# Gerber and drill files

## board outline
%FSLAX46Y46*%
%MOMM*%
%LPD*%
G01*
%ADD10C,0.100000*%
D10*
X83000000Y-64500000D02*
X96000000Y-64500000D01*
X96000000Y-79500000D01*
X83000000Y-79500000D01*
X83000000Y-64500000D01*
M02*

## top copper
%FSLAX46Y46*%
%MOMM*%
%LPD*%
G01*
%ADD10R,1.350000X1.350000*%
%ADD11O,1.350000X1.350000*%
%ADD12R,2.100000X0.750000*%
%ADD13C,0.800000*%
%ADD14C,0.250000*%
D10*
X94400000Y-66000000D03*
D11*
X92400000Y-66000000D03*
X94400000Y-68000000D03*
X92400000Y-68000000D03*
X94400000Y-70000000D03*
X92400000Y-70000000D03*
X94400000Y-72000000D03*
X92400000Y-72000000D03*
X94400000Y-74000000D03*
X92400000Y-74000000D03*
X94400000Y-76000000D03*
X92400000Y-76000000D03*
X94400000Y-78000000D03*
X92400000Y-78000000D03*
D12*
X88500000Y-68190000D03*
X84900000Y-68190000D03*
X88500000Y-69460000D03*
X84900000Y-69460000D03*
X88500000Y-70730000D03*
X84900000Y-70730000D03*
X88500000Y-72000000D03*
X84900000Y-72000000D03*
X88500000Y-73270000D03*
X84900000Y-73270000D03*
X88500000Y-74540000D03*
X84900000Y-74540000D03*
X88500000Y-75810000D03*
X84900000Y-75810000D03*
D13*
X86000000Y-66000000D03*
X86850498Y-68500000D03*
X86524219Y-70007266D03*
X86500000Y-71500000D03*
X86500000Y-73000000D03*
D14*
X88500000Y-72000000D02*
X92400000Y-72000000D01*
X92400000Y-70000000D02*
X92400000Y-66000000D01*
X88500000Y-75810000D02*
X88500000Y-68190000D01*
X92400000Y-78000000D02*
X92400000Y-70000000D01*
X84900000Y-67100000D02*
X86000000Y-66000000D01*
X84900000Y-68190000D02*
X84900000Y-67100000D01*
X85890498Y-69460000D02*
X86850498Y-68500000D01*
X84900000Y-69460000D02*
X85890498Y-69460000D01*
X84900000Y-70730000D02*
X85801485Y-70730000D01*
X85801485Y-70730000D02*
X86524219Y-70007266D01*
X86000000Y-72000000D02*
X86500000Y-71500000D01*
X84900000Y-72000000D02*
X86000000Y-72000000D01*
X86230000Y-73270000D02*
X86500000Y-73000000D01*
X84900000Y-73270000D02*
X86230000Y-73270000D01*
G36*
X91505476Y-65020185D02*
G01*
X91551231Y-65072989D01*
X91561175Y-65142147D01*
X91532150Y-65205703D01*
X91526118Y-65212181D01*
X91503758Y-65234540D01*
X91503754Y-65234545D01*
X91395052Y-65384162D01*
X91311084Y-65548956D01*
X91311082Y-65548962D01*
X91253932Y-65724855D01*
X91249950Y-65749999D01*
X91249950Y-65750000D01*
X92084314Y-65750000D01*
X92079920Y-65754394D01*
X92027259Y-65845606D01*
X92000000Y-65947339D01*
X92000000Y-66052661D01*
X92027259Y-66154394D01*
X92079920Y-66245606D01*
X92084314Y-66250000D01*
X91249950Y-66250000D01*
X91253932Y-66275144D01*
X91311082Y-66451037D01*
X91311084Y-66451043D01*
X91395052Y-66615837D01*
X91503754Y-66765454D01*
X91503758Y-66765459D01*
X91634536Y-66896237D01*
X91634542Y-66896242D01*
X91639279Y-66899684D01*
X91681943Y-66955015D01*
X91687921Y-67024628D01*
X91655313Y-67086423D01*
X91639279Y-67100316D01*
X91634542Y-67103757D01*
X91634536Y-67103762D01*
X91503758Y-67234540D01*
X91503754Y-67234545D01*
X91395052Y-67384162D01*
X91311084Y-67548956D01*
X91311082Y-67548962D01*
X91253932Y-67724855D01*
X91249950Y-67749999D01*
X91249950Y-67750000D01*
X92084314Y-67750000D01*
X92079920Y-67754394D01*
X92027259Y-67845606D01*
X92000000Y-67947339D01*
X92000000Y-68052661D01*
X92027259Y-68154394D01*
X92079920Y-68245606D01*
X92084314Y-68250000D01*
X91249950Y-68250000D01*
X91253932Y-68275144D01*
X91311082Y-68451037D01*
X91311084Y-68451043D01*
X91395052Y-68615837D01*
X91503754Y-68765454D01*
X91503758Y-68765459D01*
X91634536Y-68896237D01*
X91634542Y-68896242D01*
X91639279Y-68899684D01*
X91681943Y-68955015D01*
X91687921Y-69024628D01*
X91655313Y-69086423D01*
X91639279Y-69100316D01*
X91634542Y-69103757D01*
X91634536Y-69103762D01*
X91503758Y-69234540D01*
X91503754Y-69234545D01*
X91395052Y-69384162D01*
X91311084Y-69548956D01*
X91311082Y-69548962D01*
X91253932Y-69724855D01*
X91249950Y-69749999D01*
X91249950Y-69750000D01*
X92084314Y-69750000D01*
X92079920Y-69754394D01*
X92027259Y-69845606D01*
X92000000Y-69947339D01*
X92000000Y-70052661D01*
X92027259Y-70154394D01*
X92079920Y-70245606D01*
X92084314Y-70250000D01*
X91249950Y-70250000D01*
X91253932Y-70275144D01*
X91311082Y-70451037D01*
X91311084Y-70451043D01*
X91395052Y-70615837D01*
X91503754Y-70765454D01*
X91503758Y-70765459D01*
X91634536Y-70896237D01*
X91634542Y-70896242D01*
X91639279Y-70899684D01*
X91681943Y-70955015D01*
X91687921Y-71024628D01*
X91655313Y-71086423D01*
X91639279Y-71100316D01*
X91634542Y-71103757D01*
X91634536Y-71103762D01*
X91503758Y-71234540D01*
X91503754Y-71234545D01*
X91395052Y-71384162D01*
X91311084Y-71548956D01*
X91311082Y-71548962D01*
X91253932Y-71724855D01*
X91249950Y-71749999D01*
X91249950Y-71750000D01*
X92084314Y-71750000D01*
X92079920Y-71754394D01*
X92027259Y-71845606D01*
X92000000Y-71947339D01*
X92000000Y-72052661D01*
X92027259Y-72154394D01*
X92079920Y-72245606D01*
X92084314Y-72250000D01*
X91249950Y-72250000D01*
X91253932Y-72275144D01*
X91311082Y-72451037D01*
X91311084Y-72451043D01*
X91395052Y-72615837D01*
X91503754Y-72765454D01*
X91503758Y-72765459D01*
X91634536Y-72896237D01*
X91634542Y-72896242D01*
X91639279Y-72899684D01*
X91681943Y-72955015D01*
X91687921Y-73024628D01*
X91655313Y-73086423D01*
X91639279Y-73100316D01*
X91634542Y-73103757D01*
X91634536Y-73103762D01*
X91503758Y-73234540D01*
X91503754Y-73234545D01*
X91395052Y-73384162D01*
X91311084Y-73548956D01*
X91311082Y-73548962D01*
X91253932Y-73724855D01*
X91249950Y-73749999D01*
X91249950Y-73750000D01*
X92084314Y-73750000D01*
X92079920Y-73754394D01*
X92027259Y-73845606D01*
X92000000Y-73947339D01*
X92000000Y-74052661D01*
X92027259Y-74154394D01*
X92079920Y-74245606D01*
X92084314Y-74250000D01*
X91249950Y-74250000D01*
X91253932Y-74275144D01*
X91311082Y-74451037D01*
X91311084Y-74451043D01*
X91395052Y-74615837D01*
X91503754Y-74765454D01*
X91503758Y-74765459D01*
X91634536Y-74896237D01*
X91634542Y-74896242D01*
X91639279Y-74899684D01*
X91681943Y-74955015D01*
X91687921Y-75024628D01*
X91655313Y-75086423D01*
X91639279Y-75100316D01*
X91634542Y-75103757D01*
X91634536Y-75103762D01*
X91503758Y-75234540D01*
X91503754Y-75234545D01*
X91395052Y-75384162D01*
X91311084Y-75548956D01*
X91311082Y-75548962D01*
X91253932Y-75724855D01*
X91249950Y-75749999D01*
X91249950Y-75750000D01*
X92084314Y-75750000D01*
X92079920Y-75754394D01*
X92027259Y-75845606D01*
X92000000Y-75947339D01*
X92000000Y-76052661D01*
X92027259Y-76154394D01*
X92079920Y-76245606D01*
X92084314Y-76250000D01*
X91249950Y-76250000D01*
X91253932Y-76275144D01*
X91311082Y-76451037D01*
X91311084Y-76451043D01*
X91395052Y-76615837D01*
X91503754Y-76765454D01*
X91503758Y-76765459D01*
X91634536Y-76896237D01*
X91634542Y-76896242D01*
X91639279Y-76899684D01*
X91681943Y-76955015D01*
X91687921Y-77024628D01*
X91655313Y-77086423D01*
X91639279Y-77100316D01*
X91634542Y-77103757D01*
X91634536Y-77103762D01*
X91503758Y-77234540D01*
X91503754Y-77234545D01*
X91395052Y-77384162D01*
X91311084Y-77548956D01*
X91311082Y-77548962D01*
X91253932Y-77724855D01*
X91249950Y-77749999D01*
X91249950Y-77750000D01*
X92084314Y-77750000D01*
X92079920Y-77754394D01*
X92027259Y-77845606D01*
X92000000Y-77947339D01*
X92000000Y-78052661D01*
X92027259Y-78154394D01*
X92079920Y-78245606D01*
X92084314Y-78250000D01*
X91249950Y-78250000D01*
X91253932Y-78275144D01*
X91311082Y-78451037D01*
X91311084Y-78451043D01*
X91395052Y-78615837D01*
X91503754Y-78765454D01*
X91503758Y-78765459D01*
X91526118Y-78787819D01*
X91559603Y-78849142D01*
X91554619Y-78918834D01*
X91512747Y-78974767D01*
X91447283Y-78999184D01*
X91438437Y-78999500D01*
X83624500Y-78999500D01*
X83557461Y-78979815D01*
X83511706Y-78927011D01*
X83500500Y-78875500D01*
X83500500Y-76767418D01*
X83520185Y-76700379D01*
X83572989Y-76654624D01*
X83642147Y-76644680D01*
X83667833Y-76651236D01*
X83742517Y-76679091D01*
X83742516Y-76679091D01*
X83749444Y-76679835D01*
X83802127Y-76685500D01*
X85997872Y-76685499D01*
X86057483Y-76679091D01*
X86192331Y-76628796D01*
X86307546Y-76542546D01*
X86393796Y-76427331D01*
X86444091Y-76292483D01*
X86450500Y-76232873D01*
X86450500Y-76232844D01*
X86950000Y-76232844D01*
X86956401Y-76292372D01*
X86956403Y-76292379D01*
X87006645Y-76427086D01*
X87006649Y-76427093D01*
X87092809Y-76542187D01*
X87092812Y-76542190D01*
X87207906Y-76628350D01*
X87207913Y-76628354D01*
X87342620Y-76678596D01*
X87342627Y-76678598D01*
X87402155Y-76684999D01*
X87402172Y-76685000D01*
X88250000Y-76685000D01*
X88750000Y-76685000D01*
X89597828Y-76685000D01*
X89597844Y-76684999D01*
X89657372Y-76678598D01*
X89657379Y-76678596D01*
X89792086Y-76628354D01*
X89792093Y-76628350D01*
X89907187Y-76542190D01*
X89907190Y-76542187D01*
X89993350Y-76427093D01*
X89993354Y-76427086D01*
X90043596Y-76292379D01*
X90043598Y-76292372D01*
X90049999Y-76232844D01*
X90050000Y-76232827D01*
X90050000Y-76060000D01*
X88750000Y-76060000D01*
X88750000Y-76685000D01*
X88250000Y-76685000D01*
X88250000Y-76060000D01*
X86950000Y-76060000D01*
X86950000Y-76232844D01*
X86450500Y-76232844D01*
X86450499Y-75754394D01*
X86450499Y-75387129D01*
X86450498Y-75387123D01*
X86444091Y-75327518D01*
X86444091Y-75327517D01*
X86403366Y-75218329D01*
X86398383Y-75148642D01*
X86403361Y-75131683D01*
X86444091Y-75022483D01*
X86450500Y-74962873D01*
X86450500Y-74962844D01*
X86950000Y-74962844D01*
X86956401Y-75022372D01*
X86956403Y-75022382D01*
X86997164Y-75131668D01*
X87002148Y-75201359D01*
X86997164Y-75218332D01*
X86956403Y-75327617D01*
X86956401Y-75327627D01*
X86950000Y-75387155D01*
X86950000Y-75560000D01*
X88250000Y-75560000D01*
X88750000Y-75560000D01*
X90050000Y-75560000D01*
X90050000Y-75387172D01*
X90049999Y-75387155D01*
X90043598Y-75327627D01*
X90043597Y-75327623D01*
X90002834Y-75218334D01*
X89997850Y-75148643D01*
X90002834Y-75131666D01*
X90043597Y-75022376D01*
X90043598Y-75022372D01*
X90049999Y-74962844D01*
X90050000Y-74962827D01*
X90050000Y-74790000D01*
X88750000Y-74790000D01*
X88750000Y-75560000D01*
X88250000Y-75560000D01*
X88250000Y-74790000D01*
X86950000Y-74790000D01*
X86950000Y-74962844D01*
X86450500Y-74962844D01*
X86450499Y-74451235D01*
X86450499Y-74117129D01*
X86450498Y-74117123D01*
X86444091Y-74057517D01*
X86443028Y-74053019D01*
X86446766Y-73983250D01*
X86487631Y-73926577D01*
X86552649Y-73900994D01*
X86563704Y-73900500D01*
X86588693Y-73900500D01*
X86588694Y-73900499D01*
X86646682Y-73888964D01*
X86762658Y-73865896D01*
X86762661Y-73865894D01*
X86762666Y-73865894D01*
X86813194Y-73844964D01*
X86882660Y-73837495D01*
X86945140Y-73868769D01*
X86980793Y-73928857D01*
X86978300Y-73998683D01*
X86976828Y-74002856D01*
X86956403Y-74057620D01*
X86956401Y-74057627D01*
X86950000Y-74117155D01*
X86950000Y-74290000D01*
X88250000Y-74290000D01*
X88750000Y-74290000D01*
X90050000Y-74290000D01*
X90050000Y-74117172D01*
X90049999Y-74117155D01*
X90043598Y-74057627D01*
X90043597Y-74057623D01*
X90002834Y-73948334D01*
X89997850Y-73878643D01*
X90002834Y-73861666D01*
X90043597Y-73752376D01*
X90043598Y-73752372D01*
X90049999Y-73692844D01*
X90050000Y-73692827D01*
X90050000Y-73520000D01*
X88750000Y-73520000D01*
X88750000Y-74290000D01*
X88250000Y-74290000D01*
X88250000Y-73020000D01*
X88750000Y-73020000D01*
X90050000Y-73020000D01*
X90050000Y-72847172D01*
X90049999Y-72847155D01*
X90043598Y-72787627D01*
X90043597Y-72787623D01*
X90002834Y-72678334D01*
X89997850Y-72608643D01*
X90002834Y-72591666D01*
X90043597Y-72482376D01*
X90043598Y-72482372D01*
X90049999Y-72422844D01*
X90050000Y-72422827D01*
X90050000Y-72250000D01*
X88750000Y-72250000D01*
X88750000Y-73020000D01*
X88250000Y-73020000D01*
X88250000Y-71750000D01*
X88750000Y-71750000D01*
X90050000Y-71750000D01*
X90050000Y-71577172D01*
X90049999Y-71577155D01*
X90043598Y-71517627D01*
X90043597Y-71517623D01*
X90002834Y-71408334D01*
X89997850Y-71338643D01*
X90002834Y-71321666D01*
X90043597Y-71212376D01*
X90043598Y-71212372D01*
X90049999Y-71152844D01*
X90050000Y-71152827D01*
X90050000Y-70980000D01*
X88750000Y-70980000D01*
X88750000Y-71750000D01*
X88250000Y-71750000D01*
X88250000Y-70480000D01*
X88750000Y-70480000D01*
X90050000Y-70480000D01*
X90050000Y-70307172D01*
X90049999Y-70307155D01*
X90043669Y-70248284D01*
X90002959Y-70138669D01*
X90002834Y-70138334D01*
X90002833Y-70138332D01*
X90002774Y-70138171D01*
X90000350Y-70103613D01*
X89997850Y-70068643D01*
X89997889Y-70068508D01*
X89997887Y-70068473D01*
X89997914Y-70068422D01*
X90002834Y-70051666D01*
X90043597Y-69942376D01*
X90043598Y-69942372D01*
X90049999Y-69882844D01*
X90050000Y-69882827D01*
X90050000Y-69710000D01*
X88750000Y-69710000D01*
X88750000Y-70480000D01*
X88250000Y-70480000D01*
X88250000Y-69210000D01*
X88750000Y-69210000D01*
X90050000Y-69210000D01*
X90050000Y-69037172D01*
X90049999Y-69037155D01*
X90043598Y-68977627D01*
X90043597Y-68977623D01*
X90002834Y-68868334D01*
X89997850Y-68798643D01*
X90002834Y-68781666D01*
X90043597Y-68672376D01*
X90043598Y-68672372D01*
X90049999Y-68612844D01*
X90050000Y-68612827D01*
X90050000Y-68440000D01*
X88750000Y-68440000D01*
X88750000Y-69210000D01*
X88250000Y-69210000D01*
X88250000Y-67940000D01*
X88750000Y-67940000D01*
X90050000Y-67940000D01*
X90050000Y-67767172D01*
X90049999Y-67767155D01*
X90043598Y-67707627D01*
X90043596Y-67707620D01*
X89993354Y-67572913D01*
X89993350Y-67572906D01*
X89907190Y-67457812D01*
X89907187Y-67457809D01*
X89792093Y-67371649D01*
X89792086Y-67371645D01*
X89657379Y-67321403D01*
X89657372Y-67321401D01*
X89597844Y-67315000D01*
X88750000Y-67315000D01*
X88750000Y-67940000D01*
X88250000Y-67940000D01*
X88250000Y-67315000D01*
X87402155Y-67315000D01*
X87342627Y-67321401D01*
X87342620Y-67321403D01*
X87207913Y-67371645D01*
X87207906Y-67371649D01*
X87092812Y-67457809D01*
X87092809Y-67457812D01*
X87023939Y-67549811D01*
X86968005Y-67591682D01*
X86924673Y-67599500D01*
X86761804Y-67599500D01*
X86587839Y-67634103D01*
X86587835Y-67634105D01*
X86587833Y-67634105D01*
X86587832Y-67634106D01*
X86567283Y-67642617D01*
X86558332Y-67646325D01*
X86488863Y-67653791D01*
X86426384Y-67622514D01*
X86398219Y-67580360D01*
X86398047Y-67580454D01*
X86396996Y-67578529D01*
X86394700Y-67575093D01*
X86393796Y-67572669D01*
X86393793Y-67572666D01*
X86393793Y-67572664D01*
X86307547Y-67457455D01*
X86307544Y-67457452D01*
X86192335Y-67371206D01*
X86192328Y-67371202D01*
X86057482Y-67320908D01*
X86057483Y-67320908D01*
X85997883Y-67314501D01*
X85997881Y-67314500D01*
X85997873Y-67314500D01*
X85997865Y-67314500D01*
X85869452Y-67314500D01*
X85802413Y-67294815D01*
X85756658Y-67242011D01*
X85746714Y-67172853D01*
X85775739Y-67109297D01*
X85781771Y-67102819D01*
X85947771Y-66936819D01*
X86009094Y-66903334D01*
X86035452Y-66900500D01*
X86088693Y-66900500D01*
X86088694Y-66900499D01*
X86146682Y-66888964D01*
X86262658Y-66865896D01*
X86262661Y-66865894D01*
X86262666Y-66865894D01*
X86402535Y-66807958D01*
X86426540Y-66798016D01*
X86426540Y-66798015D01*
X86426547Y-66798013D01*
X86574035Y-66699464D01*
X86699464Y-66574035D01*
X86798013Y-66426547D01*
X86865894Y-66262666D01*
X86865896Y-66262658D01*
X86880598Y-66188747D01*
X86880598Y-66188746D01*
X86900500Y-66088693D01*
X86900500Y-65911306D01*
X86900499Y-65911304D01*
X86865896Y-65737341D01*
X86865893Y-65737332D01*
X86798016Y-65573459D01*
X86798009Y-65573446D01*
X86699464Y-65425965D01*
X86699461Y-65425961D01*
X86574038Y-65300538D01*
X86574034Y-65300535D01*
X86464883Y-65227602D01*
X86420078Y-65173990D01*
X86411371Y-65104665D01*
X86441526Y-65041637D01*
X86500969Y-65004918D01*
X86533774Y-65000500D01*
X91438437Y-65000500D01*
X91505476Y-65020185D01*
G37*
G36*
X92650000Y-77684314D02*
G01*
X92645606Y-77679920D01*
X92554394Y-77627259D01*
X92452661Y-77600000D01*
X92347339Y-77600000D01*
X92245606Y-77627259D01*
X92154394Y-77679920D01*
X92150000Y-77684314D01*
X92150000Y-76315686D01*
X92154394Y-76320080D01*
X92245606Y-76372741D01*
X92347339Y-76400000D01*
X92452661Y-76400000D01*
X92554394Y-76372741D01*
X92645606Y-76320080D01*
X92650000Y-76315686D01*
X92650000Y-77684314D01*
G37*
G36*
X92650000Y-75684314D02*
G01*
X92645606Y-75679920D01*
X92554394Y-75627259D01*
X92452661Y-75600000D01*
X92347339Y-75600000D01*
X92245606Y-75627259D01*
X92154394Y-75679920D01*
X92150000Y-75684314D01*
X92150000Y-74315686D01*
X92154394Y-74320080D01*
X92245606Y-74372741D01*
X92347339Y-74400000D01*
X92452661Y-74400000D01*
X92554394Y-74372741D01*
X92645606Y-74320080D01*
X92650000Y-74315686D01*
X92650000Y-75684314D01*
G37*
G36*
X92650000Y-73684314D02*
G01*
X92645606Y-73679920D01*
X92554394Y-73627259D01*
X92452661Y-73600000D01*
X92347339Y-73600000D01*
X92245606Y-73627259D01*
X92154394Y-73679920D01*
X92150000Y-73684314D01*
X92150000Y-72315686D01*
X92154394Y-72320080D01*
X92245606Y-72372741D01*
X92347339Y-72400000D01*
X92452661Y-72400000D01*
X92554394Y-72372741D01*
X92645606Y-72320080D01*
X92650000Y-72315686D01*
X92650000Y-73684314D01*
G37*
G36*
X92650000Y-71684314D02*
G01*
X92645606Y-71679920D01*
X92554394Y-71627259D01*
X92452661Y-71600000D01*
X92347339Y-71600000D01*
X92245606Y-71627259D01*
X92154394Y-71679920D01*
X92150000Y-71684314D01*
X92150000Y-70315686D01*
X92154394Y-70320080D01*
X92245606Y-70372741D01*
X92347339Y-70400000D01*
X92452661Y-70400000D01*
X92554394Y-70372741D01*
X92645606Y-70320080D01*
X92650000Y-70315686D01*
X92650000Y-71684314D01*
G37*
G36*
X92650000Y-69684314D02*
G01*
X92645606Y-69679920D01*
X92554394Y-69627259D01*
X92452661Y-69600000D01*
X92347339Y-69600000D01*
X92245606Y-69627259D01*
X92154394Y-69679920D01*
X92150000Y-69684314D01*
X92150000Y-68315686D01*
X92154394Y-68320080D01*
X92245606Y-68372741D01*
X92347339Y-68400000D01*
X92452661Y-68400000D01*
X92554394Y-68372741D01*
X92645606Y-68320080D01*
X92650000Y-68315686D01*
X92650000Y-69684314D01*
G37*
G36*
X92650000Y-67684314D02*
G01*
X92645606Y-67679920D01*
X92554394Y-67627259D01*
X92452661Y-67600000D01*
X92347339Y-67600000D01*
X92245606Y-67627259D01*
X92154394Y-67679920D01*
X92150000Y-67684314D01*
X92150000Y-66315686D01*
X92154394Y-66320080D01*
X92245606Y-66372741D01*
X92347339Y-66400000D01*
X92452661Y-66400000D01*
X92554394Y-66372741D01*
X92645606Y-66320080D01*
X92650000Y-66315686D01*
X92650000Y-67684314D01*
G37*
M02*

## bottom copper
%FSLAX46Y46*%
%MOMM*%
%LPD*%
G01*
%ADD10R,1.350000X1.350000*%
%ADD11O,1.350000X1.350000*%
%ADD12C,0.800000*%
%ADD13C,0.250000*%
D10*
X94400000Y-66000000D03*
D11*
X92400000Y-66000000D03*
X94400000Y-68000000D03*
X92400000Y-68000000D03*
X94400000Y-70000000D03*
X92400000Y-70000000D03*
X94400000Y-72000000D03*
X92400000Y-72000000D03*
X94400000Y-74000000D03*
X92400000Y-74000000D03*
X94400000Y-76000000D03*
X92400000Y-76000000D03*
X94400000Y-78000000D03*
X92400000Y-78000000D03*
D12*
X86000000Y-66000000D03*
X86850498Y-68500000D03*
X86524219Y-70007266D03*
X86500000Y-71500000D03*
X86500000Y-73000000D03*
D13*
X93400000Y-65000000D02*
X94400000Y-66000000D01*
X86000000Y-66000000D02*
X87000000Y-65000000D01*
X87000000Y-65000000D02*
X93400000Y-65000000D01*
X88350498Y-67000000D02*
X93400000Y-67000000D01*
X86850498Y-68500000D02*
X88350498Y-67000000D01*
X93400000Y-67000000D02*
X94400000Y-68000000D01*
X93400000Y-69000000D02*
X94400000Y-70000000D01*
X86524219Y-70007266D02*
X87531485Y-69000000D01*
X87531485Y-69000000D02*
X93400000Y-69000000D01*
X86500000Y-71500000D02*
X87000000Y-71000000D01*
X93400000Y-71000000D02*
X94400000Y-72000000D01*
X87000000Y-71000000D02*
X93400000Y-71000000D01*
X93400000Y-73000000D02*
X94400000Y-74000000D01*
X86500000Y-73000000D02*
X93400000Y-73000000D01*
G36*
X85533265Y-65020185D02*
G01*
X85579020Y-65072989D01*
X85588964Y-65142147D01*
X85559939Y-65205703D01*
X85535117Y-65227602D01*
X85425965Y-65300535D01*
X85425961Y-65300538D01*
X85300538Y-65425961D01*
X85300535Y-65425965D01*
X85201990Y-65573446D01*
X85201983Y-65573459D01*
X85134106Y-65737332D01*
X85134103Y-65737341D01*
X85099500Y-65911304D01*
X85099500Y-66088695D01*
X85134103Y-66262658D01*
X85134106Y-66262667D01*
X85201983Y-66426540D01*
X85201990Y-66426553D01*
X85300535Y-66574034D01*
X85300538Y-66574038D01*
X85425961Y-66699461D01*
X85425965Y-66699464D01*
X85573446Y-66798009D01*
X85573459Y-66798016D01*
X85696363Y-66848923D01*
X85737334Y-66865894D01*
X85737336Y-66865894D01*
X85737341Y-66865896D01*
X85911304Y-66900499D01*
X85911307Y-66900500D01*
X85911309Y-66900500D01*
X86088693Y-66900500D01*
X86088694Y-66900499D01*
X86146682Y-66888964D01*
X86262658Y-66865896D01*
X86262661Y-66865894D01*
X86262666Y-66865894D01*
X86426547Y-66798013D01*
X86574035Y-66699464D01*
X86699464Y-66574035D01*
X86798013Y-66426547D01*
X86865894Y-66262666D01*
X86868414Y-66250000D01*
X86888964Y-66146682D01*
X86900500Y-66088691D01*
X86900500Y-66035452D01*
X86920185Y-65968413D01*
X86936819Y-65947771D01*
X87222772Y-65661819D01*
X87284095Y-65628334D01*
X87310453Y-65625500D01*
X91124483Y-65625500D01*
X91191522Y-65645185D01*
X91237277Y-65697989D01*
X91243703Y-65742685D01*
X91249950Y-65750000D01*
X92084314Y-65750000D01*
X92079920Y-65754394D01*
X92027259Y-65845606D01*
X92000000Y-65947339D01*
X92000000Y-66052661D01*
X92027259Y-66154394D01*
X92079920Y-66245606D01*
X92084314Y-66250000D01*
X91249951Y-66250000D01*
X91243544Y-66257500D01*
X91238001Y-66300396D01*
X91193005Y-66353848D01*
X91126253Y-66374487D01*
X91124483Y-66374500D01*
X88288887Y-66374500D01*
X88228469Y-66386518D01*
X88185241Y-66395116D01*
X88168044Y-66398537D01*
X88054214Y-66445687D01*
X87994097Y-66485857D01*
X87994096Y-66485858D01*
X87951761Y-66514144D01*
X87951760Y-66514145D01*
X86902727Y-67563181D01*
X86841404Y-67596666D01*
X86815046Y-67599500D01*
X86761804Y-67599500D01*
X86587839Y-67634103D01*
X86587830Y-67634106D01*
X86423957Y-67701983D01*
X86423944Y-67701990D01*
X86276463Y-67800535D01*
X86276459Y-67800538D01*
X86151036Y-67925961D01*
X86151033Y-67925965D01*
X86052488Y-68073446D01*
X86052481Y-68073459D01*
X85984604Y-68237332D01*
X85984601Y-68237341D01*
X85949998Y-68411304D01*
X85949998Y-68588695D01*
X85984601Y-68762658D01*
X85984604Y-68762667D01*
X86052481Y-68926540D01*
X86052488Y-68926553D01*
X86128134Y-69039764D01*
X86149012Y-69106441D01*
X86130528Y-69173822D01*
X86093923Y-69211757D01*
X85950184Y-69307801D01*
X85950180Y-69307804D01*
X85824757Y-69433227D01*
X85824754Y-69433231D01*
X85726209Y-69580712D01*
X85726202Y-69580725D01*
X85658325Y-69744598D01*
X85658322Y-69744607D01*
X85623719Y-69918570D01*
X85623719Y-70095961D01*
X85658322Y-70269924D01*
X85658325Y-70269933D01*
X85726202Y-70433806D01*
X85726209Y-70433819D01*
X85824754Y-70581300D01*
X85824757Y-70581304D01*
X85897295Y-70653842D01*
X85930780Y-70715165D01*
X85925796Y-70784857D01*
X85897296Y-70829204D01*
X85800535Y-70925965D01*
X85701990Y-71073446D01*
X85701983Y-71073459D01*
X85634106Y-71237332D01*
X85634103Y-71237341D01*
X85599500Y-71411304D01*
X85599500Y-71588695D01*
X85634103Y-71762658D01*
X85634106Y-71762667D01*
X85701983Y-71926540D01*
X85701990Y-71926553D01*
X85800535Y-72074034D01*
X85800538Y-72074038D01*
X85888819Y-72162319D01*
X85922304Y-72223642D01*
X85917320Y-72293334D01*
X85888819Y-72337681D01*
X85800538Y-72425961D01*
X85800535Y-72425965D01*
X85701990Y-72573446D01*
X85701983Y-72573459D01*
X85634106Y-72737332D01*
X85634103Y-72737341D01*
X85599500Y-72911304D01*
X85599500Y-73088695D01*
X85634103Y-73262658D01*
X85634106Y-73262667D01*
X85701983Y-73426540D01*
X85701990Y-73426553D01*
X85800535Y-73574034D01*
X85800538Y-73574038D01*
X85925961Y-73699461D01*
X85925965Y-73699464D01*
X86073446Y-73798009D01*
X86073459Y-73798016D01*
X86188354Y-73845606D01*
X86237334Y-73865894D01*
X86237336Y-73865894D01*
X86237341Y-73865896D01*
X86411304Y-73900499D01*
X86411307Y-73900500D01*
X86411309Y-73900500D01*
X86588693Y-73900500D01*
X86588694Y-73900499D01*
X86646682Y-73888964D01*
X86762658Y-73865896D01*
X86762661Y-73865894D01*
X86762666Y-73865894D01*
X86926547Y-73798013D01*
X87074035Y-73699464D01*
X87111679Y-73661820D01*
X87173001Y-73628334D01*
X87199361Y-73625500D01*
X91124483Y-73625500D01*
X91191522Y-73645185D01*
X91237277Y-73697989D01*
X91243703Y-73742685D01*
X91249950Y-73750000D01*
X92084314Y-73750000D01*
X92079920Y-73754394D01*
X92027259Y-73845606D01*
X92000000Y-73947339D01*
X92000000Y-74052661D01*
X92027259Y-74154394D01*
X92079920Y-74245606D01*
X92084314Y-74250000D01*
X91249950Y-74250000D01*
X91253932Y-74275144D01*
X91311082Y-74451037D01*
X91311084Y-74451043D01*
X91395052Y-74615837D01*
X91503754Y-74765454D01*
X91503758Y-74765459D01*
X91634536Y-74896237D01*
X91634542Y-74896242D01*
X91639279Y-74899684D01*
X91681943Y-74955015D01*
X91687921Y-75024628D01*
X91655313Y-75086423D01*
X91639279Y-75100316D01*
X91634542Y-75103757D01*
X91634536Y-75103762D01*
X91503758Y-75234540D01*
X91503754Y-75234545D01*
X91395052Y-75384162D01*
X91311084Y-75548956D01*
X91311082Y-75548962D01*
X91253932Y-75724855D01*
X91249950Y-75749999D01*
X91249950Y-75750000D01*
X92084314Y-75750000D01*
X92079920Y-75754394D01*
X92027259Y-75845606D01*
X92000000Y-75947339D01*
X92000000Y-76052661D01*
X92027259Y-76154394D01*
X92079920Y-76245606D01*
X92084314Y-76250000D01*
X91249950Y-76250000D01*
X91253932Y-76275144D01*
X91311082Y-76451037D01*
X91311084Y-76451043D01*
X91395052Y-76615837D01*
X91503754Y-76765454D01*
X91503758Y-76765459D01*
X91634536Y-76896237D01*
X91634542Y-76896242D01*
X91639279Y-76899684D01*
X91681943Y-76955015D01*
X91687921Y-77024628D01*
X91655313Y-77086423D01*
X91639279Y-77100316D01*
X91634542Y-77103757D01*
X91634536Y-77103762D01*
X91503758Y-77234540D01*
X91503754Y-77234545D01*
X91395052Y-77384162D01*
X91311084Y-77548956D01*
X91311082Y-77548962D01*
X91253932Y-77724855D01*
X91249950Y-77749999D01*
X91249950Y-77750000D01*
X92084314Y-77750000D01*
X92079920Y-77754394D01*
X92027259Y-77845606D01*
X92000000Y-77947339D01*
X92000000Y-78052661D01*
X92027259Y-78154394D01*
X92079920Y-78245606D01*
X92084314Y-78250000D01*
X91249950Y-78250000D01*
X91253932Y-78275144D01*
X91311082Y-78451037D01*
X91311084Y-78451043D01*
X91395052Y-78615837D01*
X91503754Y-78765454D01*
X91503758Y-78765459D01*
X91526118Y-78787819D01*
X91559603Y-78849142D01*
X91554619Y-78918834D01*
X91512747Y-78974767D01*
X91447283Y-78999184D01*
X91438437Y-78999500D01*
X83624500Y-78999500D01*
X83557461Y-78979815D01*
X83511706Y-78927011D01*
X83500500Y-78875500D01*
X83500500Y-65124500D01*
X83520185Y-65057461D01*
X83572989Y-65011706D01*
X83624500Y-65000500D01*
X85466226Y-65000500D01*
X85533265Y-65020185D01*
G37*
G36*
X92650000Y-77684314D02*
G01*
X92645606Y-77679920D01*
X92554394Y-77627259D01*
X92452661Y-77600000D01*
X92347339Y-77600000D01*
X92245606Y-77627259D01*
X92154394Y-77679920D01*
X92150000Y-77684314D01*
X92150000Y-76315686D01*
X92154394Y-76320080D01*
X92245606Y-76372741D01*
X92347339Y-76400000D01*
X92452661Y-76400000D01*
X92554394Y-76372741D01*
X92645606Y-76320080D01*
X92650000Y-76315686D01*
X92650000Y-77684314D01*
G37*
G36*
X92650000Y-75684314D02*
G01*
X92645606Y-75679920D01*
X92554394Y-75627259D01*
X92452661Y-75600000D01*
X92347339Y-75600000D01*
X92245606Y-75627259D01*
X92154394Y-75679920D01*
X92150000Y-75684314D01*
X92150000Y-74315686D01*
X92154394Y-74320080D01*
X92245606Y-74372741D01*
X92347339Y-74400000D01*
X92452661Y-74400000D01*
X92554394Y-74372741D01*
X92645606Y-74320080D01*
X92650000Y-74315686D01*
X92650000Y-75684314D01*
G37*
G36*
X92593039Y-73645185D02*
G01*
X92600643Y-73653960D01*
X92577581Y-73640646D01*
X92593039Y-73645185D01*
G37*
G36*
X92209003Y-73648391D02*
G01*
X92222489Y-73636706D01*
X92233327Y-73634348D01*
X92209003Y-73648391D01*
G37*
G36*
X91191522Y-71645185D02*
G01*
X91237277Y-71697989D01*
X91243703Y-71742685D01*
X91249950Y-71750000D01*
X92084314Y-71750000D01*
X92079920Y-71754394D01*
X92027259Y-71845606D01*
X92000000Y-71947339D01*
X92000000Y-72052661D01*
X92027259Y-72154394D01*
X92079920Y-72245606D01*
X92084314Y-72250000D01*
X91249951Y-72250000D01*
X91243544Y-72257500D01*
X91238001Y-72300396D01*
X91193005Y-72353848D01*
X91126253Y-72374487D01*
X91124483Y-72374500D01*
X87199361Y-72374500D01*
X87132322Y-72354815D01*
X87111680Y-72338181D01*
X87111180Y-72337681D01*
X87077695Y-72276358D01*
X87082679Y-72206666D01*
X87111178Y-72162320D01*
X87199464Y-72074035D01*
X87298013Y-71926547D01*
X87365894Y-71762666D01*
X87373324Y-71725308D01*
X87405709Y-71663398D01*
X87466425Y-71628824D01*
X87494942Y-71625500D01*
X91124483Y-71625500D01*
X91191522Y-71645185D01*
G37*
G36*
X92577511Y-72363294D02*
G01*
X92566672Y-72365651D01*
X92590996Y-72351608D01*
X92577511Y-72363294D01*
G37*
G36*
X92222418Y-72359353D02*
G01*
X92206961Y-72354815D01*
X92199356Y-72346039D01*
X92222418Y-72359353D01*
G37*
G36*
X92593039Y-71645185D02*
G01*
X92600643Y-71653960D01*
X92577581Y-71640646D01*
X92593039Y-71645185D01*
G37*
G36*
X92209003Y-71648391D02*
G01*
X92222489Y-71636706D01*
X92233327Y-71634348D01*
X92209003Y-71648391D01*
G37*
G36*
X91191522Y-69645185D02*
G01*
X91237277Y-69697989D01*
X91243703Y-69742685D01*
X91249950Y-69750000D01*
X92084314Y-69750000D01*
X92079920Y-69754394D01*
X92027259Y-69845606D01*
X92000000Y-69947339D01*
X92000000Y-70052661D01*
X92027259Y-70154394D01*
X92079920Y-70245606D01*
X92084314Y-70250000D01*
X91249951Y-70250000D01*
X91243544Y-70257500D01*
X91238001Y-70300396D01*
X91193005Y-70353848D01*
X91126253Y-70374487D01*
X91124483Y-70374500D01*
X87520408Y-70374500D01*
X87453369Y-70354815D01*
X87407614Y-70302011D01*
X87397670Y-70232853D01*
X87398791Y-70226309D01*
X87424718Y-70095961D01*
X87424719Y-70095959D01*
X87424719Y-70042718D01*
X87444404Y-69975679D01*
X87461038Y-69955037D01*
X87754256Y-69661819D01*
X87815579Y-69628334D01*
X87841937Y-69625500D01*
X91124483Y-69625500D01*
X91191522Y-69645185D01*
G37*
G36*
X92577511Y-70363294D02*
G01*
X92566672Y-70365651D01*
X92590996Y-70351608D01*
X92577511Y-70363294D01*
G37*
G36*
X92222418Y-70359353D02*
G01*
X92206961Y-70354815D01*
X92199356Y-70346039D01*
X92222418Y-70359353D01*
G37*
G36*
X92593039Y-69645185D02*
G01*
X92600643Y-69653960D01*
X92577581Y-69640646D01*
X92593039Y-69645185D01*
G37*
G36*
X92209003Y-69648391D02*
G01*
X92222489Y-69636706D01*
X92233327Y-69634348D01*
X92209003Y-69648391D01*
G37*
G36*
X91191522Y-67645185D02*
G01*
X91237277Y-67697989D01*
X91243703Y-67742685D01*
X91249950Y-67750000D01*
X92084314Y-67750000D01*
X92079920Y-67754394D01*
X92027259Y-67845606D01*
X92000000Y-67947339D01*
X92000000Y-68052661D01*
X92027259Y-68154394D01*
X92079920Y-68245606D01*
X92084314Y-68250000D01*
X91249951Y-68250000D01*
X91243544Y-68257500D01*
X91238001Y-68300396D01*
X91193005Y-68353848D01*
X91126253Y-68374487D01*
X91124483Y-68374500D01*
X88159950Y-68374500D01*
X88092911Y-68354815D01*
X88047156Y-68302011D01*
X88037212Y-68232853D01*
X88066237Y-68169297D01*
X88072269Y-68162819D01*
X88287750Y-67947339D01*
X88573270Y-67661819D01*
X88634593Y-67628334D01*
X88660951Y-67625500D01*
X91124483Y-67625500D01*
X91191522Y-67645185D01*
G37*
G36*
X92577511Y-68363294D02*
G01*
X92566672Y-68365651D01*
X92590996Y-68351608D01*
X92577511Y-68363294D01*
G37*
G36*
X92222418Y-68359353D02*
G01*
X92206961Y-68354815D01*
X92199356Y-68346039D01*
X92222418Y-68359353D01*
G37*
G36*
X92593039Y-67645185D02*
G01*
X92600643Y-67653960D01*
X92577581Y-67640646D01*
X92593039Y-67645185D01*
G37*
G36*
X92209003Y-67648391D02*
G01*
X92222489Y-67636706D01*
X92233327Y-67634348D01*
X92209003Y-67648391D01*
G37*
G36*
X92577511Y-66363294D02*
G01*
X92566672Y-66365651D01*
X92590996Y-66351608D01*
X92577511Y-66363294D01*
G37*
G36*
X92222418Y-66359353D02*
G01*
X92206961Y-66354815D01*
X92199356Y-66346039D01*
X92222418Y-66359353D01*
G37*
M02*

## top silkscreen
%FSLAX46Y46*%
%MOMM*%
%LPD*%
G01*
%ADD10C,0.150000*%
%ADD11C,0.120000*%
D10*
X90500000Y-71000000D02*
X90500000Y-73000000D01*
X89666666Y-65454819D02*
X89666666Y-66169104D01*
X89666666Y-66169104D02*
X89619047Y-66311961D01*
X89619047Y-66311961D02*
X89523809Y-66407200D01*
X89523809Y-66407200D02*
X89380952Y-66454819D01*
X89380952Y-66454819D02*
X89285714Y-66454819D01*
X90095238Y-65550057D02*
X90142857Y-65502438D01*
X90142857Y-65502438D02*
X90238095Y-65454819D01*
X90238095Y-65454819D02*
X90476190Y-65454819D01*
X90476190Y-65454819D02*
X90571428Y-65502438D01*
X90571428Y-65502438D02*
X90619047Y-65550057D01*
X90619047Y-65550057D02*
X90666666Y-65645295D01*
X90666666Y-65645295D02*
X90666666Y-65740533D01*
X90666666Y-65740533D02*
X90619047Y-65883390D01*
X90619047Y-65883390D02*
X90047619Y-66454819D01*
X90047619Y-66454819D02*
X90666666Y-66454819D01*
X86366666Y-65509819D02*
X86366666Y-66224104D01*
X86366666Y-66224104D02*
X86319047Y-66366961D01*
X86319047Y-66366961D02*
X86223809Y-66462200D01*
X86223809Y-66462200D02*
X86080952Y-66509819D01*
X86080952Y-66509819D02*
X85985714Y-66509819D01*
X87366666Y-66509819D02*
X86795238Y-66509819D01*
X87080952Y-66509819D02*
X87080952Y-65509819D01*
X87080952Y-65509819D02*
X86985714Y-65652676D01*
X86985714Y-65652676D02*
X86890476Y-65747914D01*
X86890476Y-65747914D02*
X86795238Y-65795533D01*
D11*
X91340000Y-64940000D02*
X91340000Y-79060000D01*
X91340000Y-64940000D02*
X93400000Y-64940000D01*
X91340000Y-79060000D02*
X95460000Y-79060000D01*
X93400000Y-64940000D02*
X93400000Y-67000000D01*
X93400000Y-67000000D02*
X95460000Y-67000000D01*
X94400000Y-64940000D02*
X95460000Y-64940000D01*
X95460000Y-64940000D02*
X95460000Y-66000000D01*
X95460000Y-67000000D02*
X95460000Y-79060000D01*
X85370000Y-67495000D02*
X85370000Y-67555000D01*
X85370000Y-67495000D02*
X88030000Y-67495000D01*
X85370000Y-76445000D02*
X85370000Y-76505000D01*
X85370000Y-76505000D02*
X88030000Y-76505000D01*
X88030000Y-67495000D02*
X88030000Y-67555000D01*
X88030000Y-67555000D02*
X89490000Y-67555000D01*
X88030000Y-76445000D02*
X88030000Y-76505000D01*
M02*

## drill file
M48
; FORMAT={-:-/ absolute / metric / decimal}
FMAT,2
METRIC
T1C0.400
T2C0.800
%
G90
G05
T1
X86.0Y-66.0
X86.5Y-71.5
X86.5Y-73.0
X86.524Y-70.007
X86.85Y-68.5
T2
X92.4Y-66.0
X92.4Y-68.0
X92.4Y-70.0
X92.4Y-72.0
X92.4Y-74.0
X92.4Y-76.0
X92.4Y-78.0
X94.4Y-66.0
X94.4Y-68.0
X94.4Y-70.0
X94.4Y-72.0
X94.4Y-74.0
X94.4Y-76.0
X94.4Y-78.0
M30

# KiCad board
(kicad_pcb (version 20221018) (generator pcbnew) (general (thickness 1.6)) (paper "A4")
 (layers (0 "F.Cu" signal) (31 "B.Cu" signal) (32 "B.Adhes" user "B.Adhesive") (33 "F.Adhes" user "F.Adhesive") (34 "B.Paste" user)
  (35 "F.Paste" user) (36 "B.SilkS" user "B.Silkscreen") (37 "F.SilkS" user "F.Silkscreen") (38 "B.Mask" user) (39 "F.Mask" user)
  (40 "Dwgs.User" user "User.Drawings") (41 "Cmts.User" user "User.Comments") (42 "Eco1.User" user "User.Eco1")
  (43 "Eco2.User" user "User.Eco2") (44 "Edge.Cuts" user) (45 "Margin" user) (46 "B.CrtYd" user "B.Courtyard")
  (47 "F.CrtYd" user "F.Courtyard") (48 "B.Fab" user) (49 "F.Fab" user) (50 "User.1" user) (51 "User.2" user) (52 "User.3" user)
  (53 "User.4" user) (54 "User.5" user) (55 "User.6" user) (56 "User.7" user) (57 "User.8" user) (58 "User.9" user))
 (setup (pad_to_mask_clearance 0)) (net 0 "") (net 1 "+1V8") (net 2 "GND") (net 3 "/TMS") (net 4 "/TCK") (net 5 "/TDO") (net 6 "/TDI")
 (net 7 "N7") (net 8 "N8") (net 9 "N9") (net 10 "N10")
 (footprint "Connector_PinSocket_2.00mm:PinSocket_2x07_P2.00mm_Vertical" (layer "F.Cu") (at 94.4 66)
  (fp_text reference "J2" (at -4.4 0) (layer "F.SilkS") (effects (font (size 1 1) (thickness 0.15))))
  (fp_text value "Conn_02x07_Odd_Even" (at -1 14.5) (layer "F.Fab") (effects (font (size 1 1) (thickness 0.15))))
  (fp_line (start -3.06 -1.06) (end -3.06 13.06) (stroke (width 0.12) (type solid)) (layer "F.SilkS"))
  (fp_line (start -3.06 -1.06) (end -1 -1.06) (stroke (width 0.12) (type solid)) (layer "F.SilkS"))
  (fp_line (start -3.06 13.06) (end 1.06 13.06) (stroke (width 0.12) (type solid)) (layer "F.SilkS"))
  (fp_line (start -1 -1.06) (end -1 1) (stroke (width 0.12) (type solid)) (layer "F.SilkS"))
  (fp_line (start -1 1) (end 1.06 1) (stroke (width 0.12) (type solid)) (layer "F.SilkS"))
  (fp_line (start 0 -1.06) (end 1.06 -1.06) (stroke (width 0.12) (type solid)) (layer "F.SilkS"))
  (fp_line (start 1.06 -1.06) (end 1.06 0) (stroke (width 0.12) (type solid)) (layer "F.SilkS"))
  (fp_line (start 1.06 1) (end 1.06 13.06) (stroke (width 0.12) (type solid)) (layer "F.SilkS"))
  (pad "1" thru_hole rect (at 0 0) (size 1.35 1.35) (drill 0.8) (layers "*.Cu" "*.Mask") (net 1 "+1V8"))
  (pad "2" thru_hole oval (at -2 0) (size 1.35 1.35) (drill 0.8) (layers "*.Cu" "*.Mask") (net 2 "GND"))
  (pad "3" thru_hole oval (at 0 2) (size 1.35 1.35) (drill 0.8) (layers "*.Cu" "*.Mask") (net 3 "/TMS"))
  (pad "4" thru_hole oval (at -2 2) (size 1.35 1.35) (drill 0.8) (layers "*.Cu" "*.Mask") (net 2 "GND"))
  (pad "5" thru_hole oval (at 0 4) (size 1.35 1.35) (drill 0.8) (layers "*.Cu" "*.Mask") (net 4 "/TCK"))
  (pad "6" thru_hole oval (at -2 4) (size 1.35 1.35) (drill 0.8) (layers "*.Cu" "*.Mask") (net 2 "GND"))
  (pad "7" thru_hole oval (at 0 6) (size 1.35 1.35) (drill 0.8) (layers "*.Cu" "*.Mask") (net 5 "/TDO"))
  (pad "8" thru_hole oval (at -2 6) (size 1.35 1.35) (drill 0.8) (layers "*.Cu" "*.Mask") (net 2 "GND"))
  (pad "9" thru_hole oval (at 0 8) (size 1.35 1.35) (drill 0.8) (layers "*.Cu" "*.Mask") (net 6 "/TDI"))
  (pad "10" thru_hole oval (at -2 8) (size 1.35 1.35) (drill 0.8) (layers "*.Cu" "*.Mask") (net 2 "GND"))
  (pad "11" thru_hole oval (at 0 10) (size 1.35 1.35) (drill 0.8) (layers "*.Cu" "*.Mask") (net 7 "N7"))
  (pad "12" thru_hole oval (at -2 10) (size 1.35 1.35) (drill 0.8) (layers "*.Cu" "*.Mask") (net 2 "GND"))
  (pad "13" thru_hole oval (at 0 12) (size 1.35 1.35) (drill 0.8) (layers "*.Cu" "*.Mask") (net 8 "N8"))
  (pad "14" thru_hole oval (at -2 12) (size 1.35 1.35) (drill 0.8) (layers "*.Cu" "*.Mask") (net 2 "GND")))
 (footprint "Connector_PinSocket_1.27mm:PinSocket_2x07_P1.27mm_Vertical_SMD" (layer "F.Cu") (at 86.7 72)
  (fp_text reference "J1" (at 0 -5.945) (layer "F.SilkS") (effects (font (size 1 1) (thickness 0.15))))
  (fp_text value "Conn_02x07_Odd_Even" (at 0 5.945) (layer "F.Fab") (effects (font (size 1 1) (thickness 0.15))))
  (fp_line (start -1.33 -4.505) (end -1.33 -4.445) (stroke (width 0.12) (type solid)) (layer "F.SilkS"))
  (fp_line (start -1.33 -4.505) (end 1.33 -4.505) (stroke (width 0.12) (type solid)) (layer "F.SilkS"))
  (fp_line (start -1.33 4.445) (end -1.33 4.505) (stroke (width 0.12) (type solid)) (layer "F.SilkS"))
  (fp_line (start -1.33 4.505) (end 1.33 4.505) (stroke (width 0.12) (type solid)) (layer "F.SilkS"))
  (fp_line (start 1.33 -4.505) (end 1.33 -4.445) (stroke (width 0.12) (type solid)) (layer "F.SilkS"))
  (fp_line (start 1.33 -4.445) (end 2.79 -4.445) (stroke (width 0.12) (type solid)) (layer "F.SilkS"))
  (fp_line (start 1.33 4.445) (end 1.33 4.505) (stroke (width 0.12) (type solid)) (layer "F.SilkS"))
  (pad "1" smd rect (at 1.8 -3.81) (size 2.1 0.75) (layers "F.Cu" "F.Paste" "F.Mask") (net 2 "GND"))
  (pad "2" smd rect (at -1.8 -3.81) (size 2.1 0.75) (layers "F.Cu" "F.Paste" "F.Mask") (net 1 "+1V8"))
  (pad "3" smd rect (at 1.8 -2.54) (size 2.1 0.75) (layers "F.Cu" "F.Paste" "F.Mask") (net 2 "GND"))
  (pad "4" smd rect (at -1.8 -2.54) (size 2.1 0.75) (layers "F.Cu" "F.Paste" "F.Mask") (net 3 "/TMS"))
  (pad "5" smd rect (at 1.8 -1.27) (size 2.1 0.75) (layers "F.Cu" "F.Paste" "F.Mask") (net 2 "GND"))
  (pad "6" smd rect (at -1.8 -1.27) (size 2.1 0.75) (layers "F.Cu" "F.Paste" "F.Mask") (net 4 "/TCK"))
  (pad "7" smd rect (at 1.8 0) (size 2.1 0.75) (layers "F.Cu" "F.Paste" "F.Mask") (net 2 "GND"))
  (pad "8" smd rect (at -1.8 0) (size 2.1 0.75) (layers "F.Cu" "F.Paste" "F.Mask") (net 5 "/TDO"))
  (pad "9" smd rect (at 1.8 1.27) (size 2.1 0.75) (layers "F.Cu" "F.Paste" "F.Mask") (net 2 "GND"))
  (pad "10" smd rect (at -1.8 1.27) (size 2.1 0.75) (layers "F.Cu" "F.Paste" "F.Mask") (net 6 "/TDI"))
  (pad "11" smd rect (at 1.8 2.54) (size 2.1 0.75) (layers "F.Cu" "F.Paste" "F.Mask") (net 2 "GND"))
  (pad "12" smd rect (at -1.8 2.54) (size 2.1 0.75) (layers "F.Cu" "F.Paste" "F.Mask") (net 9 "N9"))
  (pad "13" smd rect (at 1.8 3.81) (size 2.1 0.75) (layers "F.Cu" "F.Paste" "F.Mask") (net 2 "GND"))
  (pad "14" smd rect (at -1.8 3.81) (size 2.1 0.75) (layers "F.Cu" "F.Paste" "F.Mask") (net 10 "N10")))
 (gr_line (start 90.5 71) (end 90.5 73) (stroke (width 0.15) (type default)) (layer "F.SilkS"))
 (gr_rect (start 83 64.5) (end 96 79.5) (stroke (width 0.1) (type default)) (fill none) (layer "Edge.Cuts"))
 (segment (start 88.5 72) (end 92.4 72) (width 0.25) (layer "F.Cu") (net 2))
 (segment (start 92.4 70) (end 92.4 66) (width 0.25) (layer "F.Cu") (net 2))
 (segment (start 88.5 75.81) (end 88.5 68.19) (width 0.25) (layer "F.Cu") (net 2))
 (segment (start 92.4 78) (end 92.4 70) (width 0.25) (layer "F.Cu") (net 2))
 (segment (start 84.9 67.1) (end 86 66) (width 0.25) (layer "F.Cu") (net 1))
 (segment (start 84.9 68.19) (end 84.9 67.1) (width 0.25) (layer "F.Cu") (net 1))
 (via (at 86 66) (size 0.8) (drill 0.4) (layers "F.Cu" "B.Cu") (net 1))
 (segment (start 93.4 65) (end 94.4 66) (width 0.25) (layer "B.Cu") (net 1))
 (segment (start 86 66) (end 87 65) (width 0.25) (layer "B.Cu") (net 1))
 (segment (start 87 65) (end 93.4 65) (width 0.25) (layer "B.Cu") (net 1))
 (segment (start 85.890498 69.46) (end 86.850498 68.5) (width 0.25) (layer "F.Cu") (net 3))
 (segment (start 84.9 69.46) (end 85.890498 69.46) (width 0.25) (layer "F.Cu") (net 3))
 (via (at 86.850498 68.5) (size 0.8) (drill 0.4) (layers "F.Cu" "B.Cu") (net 3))
 (segment (start 88.350498 67) (end 93.4 67) (width 0.25) (layer "B.Cu") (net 3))
 (segment (start 86.850498 68.5) (end 88.350498 67) (width 0.25) (layer "B.Cu") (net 3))
 (segment (start 93.4 67) (end 94.4 68) (width 0.25) (layer "B.Cu") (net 3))
 (segment (start 84.9 70.73) (end 85.801485 70.73) (width 0.25) (layer "F.Cu") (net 4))
 (segment (start 85.801485 70.73) (end 86.524219 70.007266) (width 0.25) (layer "F.Cu") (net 4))
 (via (at 86.524219 70.007266) (size 0.8) (drill 0.4) (layers "F.Cu" "B.Cu") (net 4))
 (segment (start 93.4 69) (end 94.4 70) (width 0.25) (layer "B.Cu") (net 4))
 (segment (start 86.524219 70.007266) (end 87.531485 69) (width 0.25) (layer "B.Cu") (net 4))
 (segment (start 87.531485 69) (end 93.4 69) (width 0.25) (layer "B.Cu") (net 4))
 (segment (start 86 72) (end 86.5 71.5) (width 0.25) (layer "F.Cu") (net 5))
 (segment (start 84.9 72) (end 86 72) (width 0.25) (layer "F.Cu") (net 5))
 (via (at 86.5 71.5) (size 0.8) (drill 0.4) (layers "F.Cu" "B.Cu") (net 5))
 (segment (start 86.5 71.5) (end 87 71) (width 0.25) (layer "B.Cu") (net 5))
 (segment (start 93.4 71) (end 94.4 72) (width 0.25) (layer "B.Cu") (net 5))
 (segment (start 87 71) (end 93.4 71) (width 0.25) (layer "B.Cu") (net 5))
 (segment (start 86.23 73.27) (end 86.5 73) (width 0.25) (layer "F.Cu") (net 6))
 (segment (start 84.9 73.27) (end 86.23 73.27) (width 0.25) (layer "F.Cu") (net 6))
 (via (at 86.5 73) (size 0.8) (drill 0.4) (layers "F.Cu" "B.Cu") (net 6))
 (segment (start 93.4 73) (end 94.4 74) (width 0.25) (layer "B.Cu") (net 6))
 (segment (start 86.5 73) (end 93.4 73) (width 0.25) (layer "B.Cu") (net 6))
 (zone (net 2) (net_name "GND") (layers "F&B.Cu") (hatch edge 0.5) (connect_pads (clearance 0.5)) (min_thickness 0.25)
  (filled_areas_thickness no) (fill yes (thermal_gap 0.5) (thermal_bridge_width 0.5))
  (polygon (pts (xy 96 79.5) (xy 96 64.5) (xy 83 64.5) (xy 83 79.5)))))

